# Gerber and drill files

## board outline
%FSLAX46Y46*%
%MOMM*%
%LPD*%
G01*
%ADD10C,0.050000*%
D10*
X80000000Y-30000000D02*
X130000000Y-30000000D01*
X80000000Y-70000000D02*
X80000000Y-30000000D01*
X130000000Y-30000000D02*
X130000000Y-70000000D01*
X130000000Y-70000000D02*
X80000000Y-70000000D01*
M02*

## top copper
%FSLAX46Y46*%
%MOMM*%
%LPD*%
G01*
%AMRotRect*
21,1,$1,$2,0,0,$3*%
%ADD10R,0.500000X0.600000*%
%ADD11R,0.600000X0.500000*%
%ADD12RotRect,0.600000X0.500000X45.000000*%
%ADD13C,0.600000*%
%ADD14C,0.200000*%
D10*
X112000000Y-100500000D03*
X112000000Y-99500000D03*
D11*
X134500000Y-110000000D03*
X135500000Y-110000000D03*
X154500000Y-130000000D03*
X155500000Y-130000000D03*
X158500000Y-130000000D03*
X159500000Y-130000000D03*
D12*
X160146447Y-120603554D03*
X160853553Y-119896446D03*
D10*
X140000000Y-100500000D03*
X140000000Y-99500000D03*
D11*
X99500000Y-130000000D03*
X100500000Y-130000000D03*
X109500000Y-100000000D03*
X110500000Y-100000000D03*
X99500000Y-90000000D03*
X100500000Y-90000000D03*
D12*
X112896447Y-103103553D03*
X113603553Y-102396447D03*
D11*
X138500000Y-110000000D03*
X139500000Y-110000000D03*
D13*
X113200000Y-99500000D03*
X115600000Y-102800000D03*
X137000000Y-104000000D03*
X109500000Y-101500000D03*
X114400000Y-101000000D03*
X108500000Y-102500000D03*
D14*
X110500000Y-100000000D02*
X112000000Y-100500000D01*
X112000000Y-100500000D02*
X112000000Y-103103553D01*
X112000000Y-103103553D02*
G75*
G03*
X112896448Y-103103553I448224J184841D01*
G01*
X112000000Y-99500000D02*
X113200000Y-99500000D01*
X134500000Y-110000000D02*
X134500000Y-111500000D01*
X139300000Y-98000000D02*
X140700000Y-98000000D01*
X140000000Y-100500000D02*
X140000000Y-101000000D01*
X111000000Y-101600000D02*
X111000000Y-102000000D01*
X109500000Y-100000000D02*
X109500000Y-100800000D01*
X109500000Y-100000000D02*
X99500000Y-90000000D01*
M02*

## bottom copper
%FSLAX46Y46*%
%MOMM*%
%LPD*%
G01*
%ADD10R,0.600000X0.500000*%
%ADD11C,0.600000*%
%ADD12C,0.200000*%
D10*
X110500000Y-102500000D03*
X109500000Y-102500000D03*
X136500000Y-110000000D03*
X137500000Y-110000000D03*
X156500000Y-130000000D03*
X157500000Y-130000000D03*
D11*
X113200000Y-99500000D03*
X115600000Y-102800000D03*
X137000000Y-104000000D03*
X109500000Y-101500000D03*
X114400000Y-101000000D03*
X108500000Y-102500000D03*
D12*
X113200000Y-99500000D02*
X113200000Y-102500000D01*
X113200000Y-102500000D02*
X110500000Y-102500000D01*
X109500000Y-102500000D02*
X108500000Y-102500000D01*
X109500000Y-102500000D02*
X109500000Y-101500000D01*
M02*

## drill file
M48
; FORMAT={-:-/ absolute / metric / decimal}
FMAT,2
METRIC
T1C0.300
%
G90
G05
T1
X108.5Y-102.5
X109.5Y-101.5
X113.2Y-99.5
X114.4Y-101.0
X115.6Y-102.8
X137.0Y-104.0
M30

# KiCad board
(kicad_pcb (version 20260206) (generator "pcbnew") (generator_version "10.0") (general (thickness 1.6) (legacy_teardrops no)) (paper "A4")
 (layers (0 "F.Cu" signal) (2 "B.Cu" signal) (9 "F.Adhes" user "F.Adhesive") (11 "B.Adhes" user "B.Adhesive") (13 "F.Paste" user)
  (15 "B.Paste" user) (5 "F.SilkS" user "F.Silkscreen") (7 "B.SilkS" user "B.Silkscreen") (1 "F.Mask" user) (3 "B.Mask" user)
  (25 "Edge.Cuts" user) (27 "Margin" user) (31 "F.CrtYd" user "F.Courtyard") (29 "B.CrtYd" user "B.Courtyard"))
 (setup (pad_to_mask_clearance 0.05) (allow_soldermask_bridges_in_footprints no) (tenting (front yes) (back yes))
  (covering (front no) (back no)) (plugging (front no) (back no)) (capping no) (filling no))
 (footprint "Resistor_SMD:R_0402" (layer "F.Cu") (at 112 100 90)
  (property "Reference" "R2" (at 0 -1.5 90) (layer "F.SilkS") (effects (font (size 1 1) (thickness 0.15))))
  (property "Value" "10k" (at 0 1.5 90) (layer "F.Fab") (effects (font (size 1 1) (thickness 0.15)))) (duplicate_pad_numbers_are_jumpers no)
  (pad "1" smd rect (at -0.5 0 90) (size 0.6 0.5) (layers "F.Cu" "F.Mask" "F.Paste") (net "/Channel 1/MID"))
  (pad "2" smd rect (at 0.5 0 90) (size 0.6 0.5) (layers "F.Cu" "F.Mask" "F.Paste") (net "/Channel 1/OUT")))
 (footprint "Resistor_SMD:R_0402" (layer "F.Cu") (at 135 110)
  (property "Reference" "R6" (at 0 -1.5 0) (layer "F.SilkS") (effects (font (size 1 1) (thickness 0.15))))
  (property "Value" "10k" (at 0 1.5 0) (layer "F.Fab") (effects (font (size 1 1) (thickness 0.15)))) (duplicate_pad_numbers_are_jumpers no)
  (pad "1" smd rect (at -0.5 0) (size 0.6 0.5) (layers "F.Cu" "F.Mask" "F.Paste") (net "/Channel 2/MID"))
  (pad "2" smd rect (at 0.5 0) (size 0.6 0.5) (layers "F.Cu" "F.Mask" "F.Paste") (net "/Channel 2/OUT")))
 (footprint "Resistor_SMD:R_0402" (layer "F.Cu") (at 155 130)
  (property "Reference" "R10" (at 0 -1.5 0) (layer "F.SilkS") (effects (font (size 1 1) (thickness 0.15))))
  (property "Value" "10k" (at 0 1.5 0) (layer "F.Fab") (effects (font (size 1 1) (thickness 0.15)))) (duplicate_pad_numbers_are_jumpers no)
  (pad "1" smd rect (at -0.5 0) (size 0.6 0.5) (layers "F.Cu" "F.Mask" "F.Paste") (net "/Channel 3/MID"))
  (pad "2" smd rect (at 0.5 0) (size 0.6 0.5) (layers "F.Cu" "F.Mask" "F.Paste") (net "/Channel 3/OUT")))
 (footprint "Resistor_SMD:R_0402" (layer "F.Cu") (at 159 130)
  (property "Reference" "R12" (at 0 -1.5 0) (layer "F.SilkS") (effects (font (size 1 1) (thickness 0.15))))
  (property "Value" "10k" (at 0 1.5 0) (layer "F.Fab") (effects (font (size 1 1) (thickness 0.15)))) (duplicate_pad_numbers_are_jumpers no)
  (pad "1" smd rect (at -0.5 0) (size 0.6 0.5) (layers "F.Cu" "F.Mask" "F.Paste") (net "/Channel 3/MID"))
  (pad "2" smd rect (at 0.5 0) (size 0.6 0.5) (layers "F.Cu" "F.Mask" "F.Paste") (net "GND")))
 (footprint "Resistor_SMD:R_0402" (layer "F.Cu") (at 160.5 120.25 45)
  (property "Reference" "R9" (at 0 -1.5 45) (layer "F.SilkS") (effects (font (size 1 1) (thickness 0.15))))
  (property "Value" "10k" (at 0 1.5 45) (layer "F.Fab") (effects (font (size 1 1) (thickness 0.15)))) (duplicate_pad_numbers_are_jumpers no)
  (pad "1" smd rect (at -0.5 0.000001 45) (size 0.6 0.5) (layers "F.Cu" "F.Mask" "F.Paste") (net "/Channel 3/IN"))
  (pad "2" smd rect (at 0.5 -0.000001 45) (size 0.6 0.5) (layers "F.Cu" "F.Mask" "F.Paste") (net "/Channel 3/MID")))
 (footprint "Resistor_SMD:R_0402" (layer "F.Cu") (at 140 100 90)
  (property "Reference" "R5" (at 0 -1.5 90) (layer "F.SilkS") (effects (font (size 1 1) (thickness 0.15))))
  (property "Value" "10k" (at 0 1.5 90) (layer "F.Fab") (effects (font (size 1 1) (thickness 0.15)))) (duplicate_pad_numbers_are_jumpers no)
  (pad "1" smd rect (at -0.5 0 90) (size 0.6 0.5) (layers "F.Cu" "F.Mask" "F.Paste") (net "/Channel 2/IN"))
  (pad "2" smd rect (at 0.5 0 90) (size 0.6 0.5) (layers "F.Cu" "F.Mask" "F.Paste") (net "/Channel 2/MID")))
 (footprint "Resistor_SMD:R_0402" (layer "F.Cu") (at 100 130)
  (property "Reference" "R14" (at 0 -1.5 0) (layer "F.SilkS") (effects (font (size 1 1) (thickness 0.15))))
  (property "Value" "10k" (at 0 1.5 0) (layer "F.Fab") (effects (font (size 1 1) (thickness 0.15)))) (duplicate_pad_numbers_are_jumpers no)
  (pad "1" smd rect (at -0.5 0) (size 0.6 0.5) (layers "F.Cu" "F.Mask" "F.Paste") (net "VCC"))
  (pad "2" smd rect (at 0.5 0) (size 0.6 0.5) (layers "F.Cu" "F.Mask" "F.Paste") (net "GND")))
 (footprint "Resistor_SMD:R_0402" (layer "F.Cu") (at 110 100)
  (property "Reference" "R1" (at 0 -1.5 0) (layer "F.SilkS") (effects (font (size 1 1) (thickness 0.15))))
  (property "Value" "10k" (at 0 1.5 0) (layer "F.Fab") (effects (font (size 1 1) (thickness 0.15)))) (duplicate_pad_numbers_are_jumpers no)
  (pad "1" smd rect (at -0.5 0) (size 0.6 0.5) (layers "F.Cu" "F.Mask" "F.Paste") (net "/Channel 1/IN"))
  (pad "2" smd rect (at 0.5 0) (size 0.6 0.5) (layers "F.Cu" "F.Mask" "F.Paste") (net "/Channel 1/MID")))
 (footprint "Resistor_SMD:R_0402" (layer "F.Cu") (at 100 90)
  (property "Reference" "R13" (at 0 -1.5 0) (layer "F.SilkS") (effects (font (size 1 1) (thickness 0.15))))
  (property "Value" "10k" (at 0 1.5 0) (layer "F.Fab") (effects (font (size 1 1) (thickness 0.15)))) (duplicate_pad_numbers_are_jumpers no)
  (pad "1" smd rect (at -0.5 0) (size 0.6 0.5) (layers "F.Cu" "F.Mask" "F.Paste") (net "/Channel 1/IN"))
  (pad "2" smd rect (at 0.5 0) (size 0.6 0.5) (layers "F.Cu" "F.Mask" "F.Paste") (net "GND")))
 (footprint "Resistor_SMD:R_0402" (layer "F.Cu") (at 113.25 102.75 45)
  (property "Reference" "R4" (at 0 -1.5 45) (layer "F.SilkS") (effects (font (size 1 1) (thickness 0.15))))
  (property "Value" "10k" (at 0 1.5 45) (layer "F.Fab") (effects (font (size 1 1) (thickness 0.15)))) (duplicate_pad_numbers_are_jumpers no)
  (pad "1" smd rect (at -0.499999 0 45) (size 0.6 0.5) (layers "F.Cu" "F.Mask" "F.Paste") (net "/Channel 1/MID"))
  (pad "2" smd rect (at 0.499999 0 45) (size 0.6 0.5) (layers "F.Cu" "F.Mask" "F.Paste") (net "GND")))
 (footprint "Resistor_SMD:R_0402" (layer "F.Cu") (at 139 110)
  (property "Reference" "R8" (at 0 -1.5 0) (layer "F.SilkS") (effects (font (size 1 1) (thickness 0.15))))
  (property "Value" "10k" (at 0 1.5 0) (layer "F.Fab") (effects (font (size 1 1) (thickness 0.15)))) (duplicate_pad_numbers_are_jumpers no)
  (pad "1" smd rect (at -0.5 0) (size 0.6 0.5) (layers "F.Cu" "F.Mask" "F.Paste") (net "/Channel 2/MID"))
  (pad "2" smd rect (at 0.5 0) (size 0.6 0.5) (layers "F.Cu" "F.Mask" "F.Paste") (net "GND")))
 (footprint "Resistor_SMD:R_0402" (layer "B.Cu") (at 110 102.5 180)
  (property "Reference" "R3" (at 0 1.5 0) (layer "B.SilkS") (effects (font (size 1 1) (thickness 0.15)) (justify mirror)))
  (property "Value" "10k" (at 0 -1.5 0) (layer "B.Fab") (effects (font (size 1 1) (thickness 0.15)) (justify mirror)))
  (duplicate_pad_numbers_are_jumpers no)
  (pad "1" smd rect (at -0.5 0 180) (size 0.6 0.5) (layers "B.Cu" "B.Mask" "B.Paste") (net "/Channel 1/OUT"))
  (pad "2" smd rect (at 0.5 0 180) (size 0.6 0.5) (layers "B.Cu" "B.Mask" "B.Paste") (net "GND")))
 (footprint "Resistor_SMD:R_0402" (layer "B.Cu") (at 137 110)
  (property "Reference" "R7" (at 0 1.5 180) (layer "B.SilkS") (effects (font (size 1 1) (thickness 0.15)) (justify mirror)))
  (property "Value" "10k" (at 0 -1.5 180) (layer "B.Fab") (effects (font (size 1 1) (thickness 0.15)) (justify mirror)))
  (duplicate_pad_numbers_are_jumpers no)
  (pad "1" smd rect (at -0.5 0) (size 0.6 0.5) (layers "B.Cu" "B.Mask" "B.Paste") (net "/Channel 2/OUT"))
  (pad "2" smd rect (at 0.5 0) (size 0.6 0.5) (layers "B.Cu" "B.Mask" "B.Paste") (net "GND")))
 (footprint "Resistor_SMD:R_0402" (layer "B.Cu") (at 157 130)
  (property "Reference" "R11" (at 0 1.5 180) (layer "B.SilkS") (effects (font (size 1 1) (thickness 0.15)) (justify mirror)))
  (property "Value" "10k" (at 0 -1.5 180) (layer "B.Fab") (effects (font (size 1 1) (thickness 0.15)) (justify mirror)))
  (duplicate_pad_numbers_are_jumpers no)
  (pad "1" smd rect (at -0.5 0) (size 0.6 0.5) (layers "B.Cu" "B.Mask" "B.Paste") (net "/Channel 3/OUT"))
  (pad "2" smd rect (at 0.5 0) (size 0.6 0.5) (layers "B.Cu" "B.Mask" "B.Paste") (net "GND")))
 (gr_line (start 80 30) (end 130 30) (stroke (width 0.05) (type default)) (layer "Edge.Cuts"))
 (gr_line (start 80 70) (end 80 30) (stroke (width 0.05) (type default)) (layer "Edge.Cuts"))
 (gr_line (start 130 30) (end 130 70) (stroke (width 0.05) (type default)) (layer "Edge.Cuts"))
 (gr_line (start 130 70) (end 80 70) (stroke (width 0.05) (type default)) (layer "Edge.Cuts"))
 (segment (start 110.5 100) (end 112 100.5) (width 0.2) (locked yes) (layer "F.Cu") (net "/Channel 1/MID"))
 (segment (start 112 100.5) (end 112 103.103553) (width 0.2) (layer "F.Cu") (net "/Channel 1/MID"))
 (arc (start 112 103.103553) (mid 112.448223 103.403553) (end 112.896447 103.103553) (width 0.2) (layer "F.Cu") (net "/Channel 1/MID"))
 (segment (start 112 99.5) (end 113.2 99.5) (width 0.2) (layer "F.Cu") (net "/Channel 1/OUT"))
 (via (at 113.2 99.5) (size 0.6) (drill 0.3) (layers "F.Cu" "B.Cu") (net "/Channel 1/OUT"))
 (segment (start 113.2 99.5) (end 113.2 102.5) (width 0.2) (layer "B.Cu") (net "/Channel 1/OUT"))
 (segment (start 113.2 102.5) (end 110.5 102.5) (width 0.2) (layer "B.Cu") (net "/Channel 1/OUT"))
 (segment (start 134.5 110) (end 134.5 111.5) (width 0.2) (layer "F.Cu") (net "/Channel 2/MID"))
 (segment (start 139.3 98) (end 140.7 98) (width 0.2) (layer "F.Cu") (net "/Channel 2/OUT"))
 (via (at 115.6 102.8) (size 0.6) (drill 0.3) (layers "F.Cu" "B.Cu") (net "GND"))
 (via (at 137 104) (size 0.6) (drill 0.3) (layers "F.Cu" "B.Cu") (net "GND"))
 (via (at 109.5 101.5) (size 0.6) (drill 0.3) (layers "F.Cu" "B.Cu") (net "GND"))
 (via (at 114.4 101) (size 0.6) (drill 0.3) (layers "F.Cu" "B.Cu") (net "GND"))
 (via (at 108.5 102.5) (size 0.6) (drill 0.3) (layers "F.Cu" "B.Cu") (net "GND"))
 (segment (start 109.5 102.5) (end 108.5 102.5) (width 0.2) (layer "B.Cu") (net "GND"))
 (segment (start 109.5 102.5) (end 109.5 101.5) (width 0.2) (layer "B.Cu") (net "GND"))
 (segment (start 140 100.5) (end 140 101) (width 0.2) (layer "F.Cu") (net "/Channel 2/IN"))
 (segment (start 111 101.6) (end 111 102) (width 0.2) (layer "F.Cu") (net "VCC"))
 (segment (start 109.5 100) (end 109.5 100.8) (width 0.2) (layer "F.Cu") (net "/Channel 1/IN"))
 (segment (start 109.5 100) (end 99.5 90) (width 0.2) (layer "F.Cu") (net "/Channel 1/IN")))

